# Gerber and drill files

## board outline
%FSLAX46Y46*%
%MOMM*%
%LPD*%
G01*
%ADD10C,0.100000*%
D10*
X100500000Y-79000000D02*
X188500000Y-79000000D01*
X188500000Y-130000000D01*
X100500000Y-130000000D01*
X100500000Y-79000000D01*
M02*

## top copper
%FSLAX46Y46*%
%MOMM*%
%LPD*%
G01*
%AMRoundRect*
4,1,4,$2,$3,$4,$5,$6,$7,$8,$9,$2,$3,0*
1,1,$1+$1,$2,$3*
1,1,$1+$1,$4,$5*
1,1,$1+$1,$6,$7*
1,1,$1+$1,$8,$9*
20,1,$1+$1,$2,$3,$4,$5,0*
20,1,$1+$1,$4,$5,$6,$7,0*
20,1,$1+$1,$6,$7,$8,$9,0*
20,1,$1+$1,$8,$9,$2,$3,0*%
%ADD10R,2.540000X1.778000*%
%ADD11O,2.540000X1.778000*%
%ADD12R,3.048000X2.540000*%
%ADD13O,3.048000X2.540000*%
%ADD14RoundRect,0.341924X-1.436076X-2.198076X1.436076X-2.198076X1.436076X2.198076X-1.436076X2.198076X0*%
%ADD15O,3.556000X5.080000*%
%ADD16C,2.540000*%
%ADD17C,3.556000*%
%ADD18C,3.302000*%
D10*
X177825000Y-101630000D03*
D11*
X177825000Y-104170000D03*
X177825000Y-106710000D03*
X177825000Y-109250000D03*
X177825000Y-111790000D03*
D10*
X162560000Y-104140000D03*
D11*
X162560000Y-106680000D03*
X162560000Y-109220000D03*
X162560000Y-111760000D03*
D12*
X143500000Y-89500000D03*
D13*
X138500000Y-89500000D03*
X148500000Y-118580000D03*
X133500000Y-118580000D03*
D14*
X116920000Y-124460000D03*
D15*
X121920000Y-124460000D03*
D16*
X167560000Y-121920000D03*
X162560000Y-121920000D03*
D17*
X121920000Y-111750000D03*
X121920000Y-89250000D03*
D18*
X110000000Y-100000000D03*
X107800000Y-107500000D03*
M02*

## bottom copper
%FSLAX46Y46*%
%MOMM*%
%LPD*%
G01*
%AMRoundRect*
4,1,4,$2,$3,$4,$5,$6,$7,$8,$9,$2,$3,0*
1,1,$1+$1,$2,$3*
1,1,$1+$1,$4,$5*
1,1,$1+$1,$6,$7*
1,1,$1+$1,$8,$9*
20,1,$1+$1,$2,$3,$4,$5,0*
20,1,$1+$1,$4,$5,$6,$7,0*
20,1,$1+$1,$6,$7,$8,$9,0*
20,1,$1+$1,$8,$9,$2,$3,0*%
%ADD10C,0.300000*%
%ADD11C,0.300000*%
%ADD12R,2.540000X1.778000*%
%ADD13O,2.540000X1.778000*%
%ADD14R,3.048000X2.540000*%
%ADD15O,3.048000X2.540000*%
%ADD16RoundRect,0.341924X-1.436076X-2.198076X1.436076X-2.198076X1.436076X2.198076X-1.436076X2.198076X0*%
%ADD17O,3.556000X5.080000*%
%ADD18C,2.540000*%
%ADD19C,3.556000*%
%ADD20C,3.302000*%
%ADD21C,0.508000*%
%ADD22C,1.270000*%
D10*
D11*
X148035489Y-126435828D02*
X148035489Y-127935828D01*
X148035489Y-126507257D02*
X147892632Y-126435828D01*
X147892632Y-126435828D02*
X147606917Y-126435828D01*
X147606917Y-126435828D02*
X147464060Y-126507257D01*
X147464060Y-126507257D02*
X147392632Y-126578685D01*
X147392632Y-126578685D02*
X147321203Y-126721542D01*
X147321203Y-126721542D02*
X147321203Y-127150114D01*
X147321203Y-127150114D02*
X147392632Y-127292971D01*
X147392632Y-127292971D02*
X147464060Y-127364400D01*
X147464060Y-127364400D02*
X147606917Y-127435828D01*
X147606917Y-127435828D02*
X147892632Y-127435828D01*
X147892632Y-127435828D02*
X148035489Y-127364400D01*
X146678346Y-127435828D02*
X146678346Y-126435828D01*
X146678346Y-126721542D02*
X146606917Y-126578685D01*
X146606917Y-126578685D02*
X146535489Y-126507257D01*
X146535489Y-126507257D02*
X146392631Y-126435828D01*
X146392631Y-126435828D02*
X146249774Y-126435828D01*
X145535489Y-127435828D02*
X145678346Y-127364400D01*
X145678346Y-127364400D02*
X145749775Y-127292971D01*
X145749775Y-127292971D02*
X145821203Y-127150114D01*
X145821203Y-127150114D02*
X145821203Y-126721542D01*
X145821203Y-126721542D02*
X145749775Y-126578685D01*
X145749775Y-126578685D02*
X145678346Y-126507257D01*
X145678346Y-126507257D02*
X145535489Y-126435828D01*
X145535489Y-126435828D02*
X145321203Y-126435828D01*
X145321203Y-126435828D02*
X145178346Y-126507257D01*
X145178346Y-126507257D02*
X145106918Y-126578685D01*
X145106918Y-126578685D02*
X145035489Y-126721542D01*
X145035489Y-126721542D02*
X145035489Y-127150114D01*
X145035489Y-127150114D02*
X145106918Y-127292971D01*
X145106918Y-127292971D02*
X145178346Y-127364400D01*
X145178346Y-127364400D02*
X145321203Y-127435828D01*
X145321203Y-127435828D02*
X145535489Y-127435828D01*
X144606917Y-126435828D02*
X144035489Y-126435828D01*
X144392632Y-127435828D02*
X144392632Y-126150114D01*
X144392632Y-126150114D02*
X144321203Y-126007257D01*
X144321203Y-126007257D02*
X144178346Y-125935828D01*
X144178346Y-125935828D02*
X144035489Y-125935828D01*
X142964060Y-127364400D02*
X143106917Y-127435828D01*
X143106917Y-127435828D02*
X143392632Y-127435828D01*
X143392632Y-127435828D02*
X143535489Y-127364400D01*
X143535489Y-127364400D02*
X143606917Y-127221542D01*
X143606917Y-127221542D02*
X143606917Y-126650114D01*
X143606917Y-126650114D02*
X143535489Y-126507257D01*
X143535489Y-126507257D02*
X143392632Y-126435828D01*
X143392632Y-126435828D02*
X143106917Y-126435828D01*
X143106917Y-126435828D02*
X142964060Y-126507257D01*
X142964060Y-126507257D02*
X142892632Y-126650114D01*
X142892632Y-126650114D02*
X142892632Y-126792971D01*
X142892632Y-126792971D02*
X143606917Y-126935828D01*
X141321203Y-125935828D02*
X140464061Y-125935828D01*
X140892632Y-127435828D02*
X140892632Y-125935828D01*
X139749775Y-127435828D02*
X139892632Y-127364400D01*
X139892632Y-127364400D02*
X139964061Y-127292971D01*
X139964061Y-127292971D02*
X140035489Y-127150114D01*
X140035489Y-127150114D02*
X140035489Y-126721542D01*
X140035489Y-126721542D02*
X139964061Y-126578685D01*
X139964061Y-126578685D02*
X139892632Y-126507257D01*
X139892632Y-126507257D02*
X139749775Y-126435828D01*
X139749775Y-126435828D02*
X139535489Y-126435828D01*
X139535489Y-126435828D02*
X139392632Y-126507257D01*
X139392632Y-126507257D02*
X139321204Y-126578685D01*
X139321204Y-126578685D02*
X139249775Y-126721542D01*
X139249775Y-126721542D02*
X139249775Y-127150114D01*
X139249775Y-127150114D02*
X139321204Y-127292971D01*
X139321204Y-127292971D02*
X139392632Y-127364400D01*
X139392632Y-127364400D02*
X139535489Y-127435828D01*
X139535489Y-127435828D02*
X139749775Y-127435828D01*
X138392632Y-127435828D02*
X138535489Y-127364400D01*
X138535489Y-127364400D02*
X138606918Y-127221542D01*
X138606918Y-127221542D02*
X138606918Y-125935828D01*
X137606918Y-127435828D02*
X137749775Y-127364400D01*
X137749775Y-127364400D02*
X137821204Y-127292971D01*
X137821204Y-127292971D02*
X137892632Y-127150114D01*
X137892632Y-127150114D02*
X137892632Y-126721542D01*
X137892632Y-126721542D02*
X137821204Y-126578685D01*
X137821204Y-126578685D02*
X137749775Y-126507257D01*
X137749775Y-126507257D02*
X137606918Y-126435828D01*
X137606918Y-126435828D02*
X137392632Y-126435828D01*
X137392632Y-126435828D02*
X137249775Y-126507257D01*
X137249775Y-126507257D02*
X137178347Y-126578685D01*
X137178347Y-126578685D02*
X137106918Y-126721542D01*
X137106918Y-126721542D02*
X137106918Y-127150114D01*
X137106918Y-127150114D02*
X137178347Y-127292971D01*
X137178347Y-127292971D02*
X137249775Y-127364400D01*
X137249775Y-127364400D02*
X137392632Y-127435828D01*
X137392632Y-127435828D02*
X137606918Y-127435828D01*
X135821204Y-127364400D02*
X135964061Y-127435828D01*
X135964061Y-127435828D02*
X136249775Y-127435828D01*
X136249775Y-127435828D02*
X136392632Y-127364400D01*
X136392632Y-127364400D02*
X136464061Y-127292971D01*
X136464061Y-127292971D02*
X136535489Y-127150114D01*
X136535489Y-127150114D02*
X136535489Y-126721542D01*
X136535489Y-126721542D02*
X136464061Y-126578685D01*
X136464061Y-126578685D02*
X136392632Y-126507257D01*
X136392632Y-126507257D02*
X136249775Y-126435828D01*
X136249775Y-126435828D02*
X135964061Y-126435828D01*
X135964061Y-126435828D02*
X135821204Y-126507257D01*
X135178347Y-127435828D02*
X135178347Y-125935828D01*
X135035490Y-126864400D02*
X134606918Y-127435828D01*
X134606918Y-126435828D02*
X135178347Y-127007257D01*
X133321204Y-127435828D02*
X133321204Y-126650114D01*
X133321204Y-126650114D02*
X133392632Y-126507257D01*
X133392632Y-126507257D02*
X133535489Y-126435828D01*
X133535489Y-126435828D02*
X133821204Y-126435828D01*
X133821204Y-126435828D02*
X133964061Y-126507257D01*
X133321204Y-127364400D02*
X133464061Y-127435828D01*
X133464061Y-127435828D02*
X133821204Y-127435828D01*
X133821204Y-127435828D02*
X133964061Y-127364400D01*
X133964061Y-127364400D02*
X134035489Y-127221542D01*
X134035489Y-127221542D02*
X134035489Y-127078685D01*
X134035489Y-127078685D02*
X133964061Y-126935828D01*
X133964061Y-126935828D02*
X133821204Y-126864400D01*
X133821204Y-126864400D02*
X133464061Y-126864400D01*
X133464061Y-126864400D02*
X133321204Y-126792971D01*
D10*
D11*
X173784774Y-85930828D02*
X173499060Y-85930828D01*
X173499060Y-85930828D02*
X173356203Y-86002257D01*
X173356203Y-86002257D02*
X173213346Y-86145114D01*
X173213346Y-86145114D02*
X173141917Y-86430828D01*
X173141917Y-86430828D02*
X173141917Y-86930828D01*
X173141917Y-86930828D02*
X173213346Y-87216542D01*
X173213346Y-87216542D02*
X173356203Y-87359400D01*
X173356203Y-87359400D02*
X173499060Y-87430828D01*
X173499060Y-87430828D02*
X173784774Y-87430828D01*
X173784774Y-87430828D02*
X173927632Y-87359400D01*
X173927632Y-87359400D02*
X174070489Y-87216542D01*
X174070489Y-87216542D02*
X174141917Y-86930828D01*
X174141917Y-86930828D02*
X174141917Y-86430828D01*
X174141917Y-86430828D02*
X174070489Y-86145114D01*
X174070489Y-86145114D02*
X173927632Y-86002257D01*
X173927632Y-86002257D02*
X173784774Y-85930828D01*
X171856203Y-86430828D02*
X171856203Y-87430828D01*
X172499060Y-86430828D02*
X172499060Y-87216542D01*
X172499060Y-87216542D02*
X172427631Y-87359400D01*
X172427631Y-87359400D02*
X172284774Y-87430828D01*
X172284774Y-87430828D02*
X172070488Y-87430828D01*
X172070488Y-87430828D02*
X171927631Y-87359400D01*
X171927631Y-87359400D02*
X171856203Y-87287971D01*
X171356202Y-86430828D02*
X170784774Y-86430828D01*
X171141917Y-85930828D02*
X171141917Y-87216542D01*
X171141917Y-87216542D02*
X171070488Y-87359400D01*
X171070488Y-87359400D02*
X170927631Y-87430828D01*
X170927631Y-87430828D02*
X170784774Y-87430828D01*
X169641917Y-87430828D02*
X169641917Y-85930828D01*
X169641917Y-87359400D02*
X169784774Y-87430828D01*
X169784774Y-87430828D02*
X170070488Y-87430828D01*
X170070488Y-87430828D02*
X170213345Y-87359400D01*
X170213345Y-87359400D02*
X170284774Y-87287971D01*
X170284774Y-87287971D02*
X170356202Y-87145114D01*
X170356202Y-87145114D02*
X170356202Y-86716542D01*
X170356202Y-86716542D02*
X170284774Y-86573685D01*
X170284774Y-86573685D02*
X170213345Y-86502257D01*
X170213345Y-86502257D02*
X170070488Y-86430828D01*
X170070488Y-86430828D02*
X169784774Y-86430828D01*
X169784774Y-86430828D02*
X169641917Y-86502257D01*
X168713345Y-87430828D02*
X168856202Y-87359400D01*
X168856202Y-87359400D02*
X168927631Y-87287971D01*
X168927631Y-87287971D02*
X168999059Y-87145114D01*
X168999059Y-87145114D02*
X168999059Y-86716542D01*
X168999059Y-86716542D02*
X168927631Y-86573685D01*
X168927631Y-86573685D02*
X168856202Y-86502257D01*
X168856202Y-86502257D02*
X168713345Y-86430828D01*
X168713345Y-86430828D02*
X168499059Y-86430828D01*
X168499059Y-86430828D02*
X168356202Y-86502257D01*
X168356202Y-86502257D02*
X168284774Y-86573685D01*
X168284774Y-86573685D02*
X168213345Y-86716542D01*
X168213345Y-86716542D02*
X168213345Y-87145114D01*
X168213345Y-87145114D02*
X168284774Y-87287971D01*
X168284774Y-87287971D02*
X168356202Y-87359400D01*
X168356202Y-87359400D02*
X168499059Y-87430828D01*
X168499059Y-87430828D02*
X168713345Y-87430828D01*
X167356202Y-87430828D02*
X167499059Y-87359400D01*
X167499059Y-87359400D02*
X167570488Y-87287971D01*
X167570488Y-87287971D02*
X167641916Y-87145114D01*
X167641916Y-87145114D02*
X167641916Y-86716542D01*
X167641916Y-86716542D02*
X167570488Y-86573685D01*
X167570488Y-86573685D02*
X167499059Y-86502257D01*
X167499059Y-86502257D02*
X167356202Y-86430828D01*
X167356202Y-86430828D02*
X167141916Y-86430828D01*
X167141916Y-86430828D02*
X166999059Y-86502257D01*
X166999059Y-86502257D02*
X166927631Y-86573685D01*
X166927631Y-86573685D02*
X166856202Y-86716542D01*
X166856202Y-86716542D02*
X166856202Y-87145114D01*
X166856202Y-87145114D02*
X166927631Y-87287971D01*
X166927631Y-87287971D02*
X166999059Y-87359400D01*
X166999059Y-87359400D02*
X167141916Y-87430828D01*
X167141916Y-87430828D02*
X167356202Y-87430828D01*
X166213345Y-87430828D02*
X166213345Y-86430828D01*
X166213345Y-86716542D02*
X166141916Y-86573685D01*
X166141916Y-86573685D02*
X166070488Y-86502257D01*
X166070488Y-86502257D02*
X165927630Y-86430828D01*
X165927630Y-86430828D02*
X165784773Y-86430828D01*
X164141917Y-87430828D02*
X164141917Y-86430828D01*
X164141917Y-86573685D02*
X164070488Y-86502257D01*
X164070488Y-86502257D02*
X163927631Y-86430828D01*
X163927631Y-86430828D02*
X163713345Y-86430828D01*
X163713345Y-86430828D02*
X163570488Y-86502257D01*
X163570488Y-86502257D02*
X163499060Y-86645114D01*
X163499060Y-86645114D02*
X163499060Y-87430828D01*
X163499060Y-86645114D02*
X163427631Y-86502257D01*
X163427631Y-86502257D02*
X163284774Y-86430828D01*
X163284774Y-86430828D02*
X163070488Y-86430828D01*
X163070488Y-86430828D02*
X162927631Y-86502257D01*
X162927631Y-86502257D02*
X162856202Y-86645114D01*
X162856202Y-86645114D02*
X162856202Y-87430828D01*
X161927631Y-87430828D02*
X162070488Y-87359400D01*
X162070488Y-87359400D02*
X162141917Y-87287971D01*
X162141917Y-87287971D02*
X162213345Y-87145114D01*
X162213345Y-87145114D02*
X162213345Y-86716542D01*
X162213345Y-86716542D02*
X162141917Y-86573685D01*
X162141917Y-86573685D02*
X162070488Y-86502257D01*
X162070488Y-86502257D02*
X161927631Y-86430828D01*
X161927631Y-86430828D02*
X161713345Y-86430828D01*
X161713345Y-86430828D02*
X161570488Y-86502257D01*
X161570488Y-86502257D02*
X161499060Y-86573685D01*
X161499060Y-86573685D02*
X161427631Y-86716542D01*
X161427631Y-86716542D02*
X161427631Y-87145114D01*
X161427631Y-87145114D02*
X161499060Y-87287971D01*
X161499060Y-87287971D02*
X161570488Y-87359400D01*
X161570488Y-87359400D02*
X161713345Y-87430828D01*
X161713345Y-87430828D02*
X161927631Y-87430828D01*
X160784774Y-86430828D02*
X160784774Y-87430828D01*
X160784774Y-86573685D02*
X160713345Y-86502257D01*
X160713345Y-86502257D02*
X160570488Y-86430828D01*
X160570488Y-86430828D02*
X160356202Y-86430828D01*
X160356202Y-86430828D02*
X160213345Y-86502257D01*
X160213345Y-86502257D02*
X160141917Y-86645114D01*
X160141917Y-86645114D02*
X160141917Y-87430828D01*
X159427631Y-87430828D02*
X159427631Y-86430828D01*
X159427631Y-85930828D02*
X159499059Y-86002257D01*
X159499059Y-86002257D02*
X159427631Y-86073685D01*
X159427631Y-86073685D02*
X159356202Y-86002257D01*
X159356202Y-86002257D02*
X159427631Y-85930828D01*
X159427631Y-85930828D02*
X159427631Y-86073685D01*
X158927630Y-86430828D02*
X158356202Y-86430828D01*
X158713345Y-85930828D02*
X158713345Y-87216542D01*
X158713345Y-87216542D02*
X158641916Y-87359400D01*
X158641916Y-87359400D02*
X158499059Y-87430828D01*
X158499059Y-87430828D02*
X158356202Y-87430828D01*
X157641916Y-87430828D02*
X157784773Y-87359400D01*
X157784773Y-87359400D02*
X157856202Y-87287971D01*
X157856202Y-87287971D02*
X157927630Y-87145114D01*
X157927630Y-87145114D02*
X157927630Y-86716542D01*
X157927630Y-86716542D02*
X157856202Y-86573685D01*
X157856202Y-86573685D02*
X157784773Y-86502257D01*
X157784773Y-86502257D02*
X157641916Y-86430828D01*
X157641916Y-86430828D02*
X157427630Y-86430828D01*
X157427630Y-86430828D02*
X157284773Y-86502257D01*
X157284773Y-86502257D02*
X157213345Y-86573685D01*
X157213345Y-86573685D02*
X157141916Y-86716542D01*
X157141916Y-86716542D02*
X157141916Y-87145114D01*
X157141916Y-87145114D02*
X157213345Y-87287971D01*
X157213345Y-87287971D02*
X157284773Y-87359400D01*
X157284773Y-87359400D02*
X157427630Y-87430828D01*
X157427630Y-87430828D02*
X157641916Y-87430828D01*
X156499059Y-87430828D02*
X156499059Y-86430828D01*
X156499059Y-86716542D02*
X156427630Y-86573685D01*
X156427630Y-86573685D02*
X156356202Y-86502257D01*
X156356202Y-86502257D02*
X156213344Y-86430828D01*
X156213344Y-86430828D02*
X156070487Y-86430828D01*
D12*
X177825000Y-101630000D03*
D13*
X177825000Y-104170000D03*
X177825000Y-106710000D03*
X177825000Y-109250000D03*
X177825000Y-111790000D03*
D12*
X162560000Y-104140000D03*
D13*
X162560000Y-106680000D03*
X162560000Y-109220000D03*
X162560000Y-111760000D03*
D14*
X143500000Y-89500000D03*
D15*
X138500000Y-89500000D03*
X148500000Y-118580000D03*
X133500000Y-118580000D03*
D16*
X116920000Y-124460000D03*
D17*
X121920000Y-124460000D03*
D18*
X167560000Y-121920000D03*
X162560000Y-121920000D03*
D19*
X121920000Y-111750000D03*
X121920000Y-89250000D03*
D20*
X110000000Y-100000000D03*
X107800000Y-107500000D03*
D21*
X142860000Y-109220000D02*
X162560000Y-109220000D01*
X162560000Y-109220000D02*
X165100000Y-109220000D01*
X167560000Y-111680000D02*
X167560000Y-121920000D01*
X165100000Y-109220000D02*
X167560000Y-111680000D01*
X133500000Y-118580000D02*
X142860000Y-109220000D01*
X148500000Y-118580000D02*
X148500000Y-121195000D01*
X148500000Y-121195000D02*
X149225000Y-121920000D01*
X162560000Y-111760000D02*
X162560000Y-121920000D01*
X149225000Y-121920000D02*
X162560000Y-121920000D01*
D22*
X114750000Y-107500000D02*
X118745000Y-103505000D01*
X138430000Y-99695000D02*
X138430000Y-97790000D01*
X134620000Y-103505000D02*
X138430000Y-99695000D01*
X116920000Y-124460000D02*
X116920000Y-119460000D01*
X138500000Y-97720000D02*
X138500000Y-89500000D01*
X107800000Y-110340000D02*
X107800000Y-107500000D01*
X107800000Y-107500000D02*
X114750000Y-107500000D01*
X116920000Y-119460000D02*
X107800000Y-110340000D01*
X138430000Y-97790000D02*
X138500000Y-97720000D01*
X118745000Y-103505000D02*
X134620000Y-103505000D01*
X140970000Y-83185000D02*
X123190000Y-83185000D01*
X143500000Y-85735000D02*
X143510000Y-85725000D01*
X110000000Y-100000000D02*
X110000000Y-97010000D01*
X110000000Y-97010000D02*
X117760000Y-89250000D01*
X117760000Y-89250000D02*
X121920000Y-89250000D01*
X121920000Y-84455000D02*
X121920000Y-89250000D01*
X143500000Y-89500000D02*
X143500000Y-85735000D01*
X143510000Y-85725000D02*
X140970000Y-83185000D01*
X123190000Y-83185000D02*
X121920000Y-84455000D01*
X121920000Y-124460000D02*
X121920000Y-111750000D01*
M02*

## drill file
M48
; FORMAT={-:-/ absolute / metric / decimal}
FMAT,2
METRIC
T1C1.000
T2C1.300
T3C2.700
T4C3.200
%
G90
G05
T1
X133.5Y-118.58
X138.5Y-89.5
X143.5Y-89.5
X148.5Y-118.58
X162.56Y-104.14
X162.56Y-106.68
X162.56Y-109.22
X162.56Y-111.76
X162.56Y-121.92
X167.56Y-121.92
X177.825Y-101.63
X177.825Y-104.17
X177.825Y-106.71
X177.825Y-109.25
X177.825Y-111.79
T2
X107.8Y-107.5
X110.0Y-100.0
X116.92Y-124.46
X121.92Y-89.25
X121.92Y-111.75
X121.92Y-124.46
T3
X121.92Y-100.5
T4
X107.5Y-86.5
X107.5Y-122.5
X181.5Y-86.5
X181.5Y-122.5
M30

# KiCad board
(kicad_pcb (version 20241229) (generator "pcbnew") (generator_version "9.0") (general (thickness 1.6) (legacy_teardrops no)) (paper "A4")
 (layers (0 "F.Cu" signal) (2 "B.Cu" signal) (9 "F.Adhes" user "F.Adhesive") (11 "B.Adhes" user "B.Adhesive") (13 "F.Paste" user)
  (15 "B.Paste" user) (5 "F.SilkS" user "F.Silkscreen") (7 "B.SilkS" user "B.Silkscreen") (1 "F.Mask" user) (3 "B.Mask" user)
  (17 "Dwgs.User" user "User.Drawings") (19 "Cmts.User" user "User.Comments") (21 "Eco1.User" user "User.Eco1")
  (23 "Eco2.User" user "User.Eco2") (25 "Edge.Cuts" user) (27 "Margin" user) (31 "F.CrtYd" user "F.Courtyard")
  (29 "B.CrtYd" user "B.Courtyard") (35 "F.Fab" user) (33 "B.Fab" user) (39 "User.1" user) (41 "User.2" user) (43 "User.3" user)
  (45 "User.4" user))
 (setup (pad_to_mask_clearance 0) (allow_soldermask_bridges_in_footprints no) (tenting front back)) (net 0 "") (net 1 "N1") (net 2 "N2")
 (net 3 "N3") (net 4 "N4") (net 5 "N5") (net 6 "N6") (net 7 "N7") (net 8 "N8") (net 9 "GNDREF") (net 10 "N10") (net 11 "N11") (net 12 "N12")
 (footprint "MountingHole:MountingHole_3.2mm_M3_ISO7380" (layer "F.Cu") (at 181.5 122.5)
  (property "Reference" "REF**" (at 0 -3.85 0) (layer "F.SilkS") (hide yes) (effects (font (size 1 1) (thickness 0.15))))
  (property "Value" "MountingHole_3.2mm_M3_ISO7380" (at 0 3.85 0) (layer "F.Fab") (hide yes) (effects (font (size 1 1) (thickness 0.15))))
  (pad "" np_thru_hole circle (at 0 0) (size 3.2 3.2) (drill 3.2) (layers "*.Cu" "*.Mask")))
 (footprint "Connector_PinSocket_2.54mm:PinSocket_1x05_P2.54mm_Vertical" (layer "F.Cu") (at 177.825 101.63)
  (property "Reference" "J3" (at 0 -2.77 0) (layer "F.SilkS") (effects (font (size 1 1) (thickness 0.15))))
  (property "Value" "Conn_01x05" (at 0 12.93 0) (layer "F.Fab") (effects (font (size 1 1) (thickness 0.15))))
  (pad "1" thru_hole rect (at 0 0) (size 2.54 1.778) (drill 1) (layers "*.Cu" "*.Mask") (remove_unused_layers no) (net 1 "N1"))
  (pad "2" thru_hole oval (at 0 2.54) (size 2.54 1.778) (drill 1) (layers "*.Cu" "*.Mask") (remove_unused_layers no) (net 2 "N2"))
  (pad "3" thru_hole oval (at 0 5.08) (size 2.54 1.778) (drill 1) (layers "*.Cu" "*.Mask") (remove_unused_layers no) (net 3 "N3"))
  (pad "4" thru_hole oval (at 0 7.62) (size 2.54 1.778) (drill 1) (layers "*.Cu" "*.Mask") (remove_unused_layers no) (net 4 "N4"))
  (pad "5" thru_hole oval (at 0 10.16) (size 2.54 1.778) (drill 1) (layers "*.Cu" "*.Mask") (remove_unused_layers no) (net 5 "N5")))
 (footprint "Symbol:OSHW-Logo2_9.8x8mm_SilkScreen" (layer "F.Cu") (at 165.1 85.09)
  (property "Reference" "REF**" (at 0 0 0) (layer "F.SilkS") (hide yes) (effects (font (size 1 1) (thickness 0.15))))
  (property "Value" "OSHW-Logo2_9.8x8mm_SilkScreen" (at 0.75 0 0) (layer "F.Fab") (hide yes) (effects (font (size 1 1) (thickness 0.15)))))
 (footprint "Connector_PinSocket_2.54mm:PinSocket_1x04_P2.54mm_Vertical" (layer "F.Cu") (at 162.56 104.14)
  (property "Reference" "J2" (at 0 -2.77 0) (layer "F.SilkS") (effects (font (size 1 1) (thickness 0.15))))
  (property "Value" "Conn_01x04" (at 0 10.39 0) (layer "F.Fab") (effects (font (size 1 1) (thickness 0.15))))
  (pad "1" thru_hole rect (at 0 0) (size 2.54 1.778) (drill 1) (layers "*.Cu" "*.Mask") (remove_unused_layers no) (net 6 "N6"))
  (pad "2" thru_hole oval (at 0 2.54) (size 2.54 1.778) (drill 1) (layers "*.Cu" "*.Mask") (remove_unused_layers no) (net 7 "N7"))
  (pad "3" thru_hole oval (at 0 5.08) (size 2.54 1.778) (drill 1) (layers "*.Cu" "*.Mask") (remove_unused_layers no) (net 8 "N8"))
  (pad "4" thru_hole oval (at 0 7.62) (size 2.54 1.778) (drill 1) (layers "*.Cu" "*.Mask") (remove_unused_layers no) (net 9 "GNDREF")))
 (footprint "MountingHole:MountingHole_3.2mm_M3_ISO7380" (layer "F.Cu") (at 107.5 86.5)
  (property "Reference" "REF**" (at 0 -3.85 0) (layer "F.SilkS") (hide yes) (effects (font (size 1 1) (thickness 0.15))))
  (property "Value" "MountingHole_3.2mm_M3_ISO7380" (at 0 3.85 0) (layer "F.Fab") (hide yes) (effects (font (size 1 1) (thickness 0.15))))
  (pad "" np_thru_hole circle (at 0 0) (size 3.2 3.2) (drill 3.2) (layers "*.Cu" "*.Mask")))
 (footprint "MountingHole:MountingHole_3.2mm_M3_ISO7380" (layer "F.Cu") (at 107.5 122.5)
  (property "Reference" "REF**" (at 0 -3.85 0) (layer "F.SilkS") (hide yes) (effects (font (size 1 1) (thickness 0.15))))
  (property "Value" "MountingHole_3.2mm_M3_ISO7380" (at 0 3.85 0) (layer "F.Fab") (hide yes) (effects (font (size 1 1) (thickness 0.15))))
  (pad "" np_thru_hole circle (at 0 0) (size 3.2 3.2) (drill 3.2) (layers "*.Cu" "*.Mask")))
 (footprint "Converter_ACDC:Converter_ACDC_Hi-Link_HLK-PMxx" (layer "F.Cu") (at 143.5 89.5 -90)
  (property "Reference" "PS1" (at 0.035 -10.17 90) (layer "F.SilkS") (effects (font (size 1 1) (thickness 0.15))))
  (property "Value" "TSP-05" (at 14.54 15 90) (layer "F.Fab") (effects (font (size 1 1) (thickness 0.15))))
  (pad "1" thru_hole rect (at 0 0 270) (size 2.54 3.048) (drill 1) (layers "*.Cu" "*.Mask") (remove_unused_layers no) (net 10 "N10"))
  (pad "2" thru_hole oval (at 0 5 270) (size 2.54 3.048) (drill 1) (layers "*.Cu" "*.Mask") (remove_unused_layers no) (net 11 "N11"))
  (pad "3" thru_hole oval (at 29.08 -5 270) (size 2.54 3.048) (drill 1) (layers "*.Cu" "*.Mask") (remove_unused_layers no) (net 9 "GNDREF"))
  (pad "4" thru_hole oval (at 29.08 10 270) (size 2.54 3.048) (drill 1) (layers "*.Cu" "*.Mask") (remove_unused_layers no) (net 8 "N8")))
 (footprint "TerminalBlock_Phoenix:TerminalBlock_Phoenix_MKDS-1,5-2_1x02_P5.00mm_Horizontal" (layer "F.Cu") (at 116.92 124.46)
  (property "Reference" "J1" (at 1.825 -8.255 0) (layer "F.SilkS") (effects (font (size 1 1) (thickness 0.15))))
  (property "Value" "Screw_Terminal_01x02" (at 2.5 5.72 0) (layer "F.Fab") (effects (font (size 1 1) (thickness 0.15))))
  (pad "1" thru_hole roundrect (at 0 0) (size 3.556 5.08) (drill 1.3) (layers "*.Cu" "*.Mask") (remove_unused_layers no)
   (roundrect_rratio 0.096154) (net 11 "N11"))
  (pad "2" thru_hole oval (at 5 0) (size 3.556 5.08) (drill 1.3) (layers "*.Cu" "*.Mask") (remove_unused_layers no) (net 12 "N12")))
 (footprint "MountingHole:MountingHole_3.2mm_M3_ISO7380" (layer "F.Cu") (at 181.5 86.5)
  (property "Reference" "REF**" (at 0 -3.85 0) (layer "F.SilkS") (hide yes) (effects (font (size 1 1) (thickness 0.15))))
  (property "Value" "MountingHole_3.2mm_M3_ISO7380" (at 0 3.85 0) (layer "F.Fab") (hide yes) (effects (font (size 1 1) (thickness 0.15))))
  (pad "" np_thru_hole circle (at 0 0) (size 3.2 3.2) (drill 3.2) (layers "*.Cu" "*.Mask")))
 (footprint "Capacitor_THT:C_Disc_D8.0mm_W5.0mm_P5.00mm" (layer "F.Cu") (at 167.56 121.92 180)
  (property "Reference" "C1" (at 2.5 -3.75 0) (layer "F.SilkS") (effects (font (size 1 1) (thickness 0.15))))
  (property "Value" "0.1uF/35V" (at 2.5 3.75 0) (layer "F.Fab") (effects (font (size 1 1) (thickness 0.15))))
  (pad "1" thru_hole circle (at 0 0 180) (size 2.54 2.54) (drill 1) (layers "*.Cu" "*.Mask") (remove_unused_layers no) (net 8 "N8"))
  (pad "2" thru_hole circle (at 5 0 180) (size 2.54 2.54) (drill 1) (layers "*.Cu" "*.Mask") (remove_unused_layers no) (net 9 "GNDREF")))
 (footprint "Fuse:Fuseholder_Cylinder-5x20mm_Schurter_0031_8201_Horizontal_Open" (layer "F.Cu") (at 121.92 111.75 90)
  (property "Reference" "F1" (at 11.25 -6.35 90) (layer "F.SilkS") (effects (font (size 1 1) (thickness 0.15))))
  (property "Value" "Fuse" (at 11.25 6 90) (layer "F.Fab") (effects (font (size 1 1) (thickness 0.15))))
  (pad "" np_thru_hole circle (at 11.25 0 90) (size 2.7 2.7) (drill 2.7) (layers "*.Cu" "*.Mask"))
  (pad "1" thru_hole circle (at 0 0 90) (size 3.556 3.556) (drill 1.3) (layers "*.Cu" "*.Mask") (remove_unused_layers no) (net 12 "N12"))
  (pad "2" thru_hole circle (at 22.5 0 90) (size 3.556 3.556) (drill 1.3) (layers "*.Cu" "*.Mask") (remove_unused_layers no) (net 10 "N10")))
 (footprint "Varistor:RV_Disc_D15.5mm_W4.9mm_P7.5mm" (layer "F.Cu") (at 110 100 -90)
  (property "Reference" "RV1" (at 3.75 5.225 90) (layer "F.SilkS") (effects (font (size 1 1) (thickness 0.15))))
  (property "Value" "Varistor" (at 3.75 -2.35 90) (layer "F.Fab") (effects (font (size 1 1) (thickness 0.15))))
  (pad "1" thru_hole circle (at 0 0 270) (size 3.302 3.302) (drill 1.3) (layers "*.Cu" "*.Mask") (remove_unused_layers no) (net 10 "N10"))
  (pad "2" thru_hole circle (at 7.5 2.2 270) (size 3.302 3.302) (drill 1.3) (layers "*.Cu" "*.Mask") (remove_unused_layers no)
   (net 11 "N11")))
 (gr_rect (start 100.5 79) (end 188.5 130) (stroke (width 0.1) (type solid)) (fill no) (layer "Edge.Cuts"))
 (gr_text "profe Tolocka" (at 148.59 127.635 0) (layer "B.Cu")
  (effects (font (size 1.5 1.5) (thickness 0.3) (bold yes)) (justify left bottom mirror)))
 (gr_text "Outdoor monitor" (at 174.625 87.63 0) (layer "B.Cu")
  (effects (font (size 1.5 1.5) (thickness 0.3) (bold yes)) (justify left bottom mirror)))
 (segment (start 142.86 109.22) (end 162.56 109.22) (width 0.508) (layer "B.Cu") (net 8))
 (segment (start 162.56 109.22) (end 165.1 109.22) (width 0.508) (layer "B.Cu") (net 8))
 (segment (start 167.56 111.68) (end 167.56 121.92) (width 0.508) (layer "B.Cu") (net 8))
 (segment (start 165.1 109.22) (end 167.56 111.68) (width 0.508) (layer "B.Cu") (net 8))
 (segment (start 133.5 118.58) (end 142.86 109.22) (width 0.508) (layer "B.Cu") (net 8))
 (segment (start 148.5 118.58) (end 148.5 121.195) (width 0.508) (layer "B.Cu") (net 9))
 (segment (start 148.5 121.195) (end 149.225 121.92) (width 0.508) (layer "B.Cu") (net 9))
 (segment (start 162.56 111.76) (end 162.56 121.92) (width 0.508) (layer "B.Cu") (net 9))
 (segment (start 149.225 121.92) (end 162.56 121.92) (width 0.508) (layer "B.Cu") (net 9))
 (segment (start 114.75 107.5) (end 118.745 103.505) (width 1.27) (layer "B.Cu") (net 11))
 (segment (start 138.43 99.695) (end 138.43 97.79) (width 1.27) (layer "B.Cu") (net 11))
 (segment (start 134.62 103.505) (end 138.43 99.695) (width 1.27) (layer "B.Cu") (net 11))
 (segment (start 116.92 124.46) (end 116.92 119.46) (width 1.27) (layer "B.Cu") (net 11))
 (segment (start 138.5 97.72) (end 138.5 89.5) (width 1.27) (layer "B.Cu") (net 11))
 (segment (start 107.8 110.34) (end 107.8 107.5) (width 1.27) (layer "B.Cu") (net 11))
 (segment (start 107.8 107.5) (end 114.75 107.5) (width 1.27) (layer "B.Cu") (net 11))
 (segment (start 116.92 119.46) (end 107.8 110.34) (width 1.27) (layer "B.Cu") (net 11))
 (segment (start 138.43 97.79) (end 138.5 97.72) (width 1.27) (layer "B.Cu") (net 11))
 (segment (start 118.745 103.505) (end 134.62 103.505) (width 1.27) (layer "B.Cu") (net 11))
 (segment (start 140.97 83.185) (end 123.19 83.185) (width 1.27) (layer "B.Cu") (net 10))
 (segment (start 143.5 85.735) (end 143.51 85.725) (width 1.27) (layer "B.Cu") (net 10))
 (segment (start 110 100) (end 110 97.01) (width 1.27) (layer "B.Cu") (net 10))
 (segment (start 110 97.01) (end 117.76 89.25) (width 1.27) (layer "B.Cu") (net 10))
 (segment (start 117.76 89.25) (end 121.92 89.25) (width 1.27) (layer "B.Cu") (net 10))
 (segment (start 121.92 84.455) (end 121.92 89.25) (width 1.27) (layer "B.Cu") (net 10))
 (segment (start 143.5 89.5) (end 143.5 85.735) (width 1.27) (layer "B.Cu") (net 10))
 (segment (start 143.51 85.725) (end 140.97 83.185) (width 1.27) (layer "B.Cu") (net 10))
 (segment (start 123.19 83.185) (end 121.92 84.455) (width 1.27) (layer "B.Cu") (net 10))
 (segment (start 121.92 124.46) (end 121.92 111.75) (width 1.27) (layer "B.Cu") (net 12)))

